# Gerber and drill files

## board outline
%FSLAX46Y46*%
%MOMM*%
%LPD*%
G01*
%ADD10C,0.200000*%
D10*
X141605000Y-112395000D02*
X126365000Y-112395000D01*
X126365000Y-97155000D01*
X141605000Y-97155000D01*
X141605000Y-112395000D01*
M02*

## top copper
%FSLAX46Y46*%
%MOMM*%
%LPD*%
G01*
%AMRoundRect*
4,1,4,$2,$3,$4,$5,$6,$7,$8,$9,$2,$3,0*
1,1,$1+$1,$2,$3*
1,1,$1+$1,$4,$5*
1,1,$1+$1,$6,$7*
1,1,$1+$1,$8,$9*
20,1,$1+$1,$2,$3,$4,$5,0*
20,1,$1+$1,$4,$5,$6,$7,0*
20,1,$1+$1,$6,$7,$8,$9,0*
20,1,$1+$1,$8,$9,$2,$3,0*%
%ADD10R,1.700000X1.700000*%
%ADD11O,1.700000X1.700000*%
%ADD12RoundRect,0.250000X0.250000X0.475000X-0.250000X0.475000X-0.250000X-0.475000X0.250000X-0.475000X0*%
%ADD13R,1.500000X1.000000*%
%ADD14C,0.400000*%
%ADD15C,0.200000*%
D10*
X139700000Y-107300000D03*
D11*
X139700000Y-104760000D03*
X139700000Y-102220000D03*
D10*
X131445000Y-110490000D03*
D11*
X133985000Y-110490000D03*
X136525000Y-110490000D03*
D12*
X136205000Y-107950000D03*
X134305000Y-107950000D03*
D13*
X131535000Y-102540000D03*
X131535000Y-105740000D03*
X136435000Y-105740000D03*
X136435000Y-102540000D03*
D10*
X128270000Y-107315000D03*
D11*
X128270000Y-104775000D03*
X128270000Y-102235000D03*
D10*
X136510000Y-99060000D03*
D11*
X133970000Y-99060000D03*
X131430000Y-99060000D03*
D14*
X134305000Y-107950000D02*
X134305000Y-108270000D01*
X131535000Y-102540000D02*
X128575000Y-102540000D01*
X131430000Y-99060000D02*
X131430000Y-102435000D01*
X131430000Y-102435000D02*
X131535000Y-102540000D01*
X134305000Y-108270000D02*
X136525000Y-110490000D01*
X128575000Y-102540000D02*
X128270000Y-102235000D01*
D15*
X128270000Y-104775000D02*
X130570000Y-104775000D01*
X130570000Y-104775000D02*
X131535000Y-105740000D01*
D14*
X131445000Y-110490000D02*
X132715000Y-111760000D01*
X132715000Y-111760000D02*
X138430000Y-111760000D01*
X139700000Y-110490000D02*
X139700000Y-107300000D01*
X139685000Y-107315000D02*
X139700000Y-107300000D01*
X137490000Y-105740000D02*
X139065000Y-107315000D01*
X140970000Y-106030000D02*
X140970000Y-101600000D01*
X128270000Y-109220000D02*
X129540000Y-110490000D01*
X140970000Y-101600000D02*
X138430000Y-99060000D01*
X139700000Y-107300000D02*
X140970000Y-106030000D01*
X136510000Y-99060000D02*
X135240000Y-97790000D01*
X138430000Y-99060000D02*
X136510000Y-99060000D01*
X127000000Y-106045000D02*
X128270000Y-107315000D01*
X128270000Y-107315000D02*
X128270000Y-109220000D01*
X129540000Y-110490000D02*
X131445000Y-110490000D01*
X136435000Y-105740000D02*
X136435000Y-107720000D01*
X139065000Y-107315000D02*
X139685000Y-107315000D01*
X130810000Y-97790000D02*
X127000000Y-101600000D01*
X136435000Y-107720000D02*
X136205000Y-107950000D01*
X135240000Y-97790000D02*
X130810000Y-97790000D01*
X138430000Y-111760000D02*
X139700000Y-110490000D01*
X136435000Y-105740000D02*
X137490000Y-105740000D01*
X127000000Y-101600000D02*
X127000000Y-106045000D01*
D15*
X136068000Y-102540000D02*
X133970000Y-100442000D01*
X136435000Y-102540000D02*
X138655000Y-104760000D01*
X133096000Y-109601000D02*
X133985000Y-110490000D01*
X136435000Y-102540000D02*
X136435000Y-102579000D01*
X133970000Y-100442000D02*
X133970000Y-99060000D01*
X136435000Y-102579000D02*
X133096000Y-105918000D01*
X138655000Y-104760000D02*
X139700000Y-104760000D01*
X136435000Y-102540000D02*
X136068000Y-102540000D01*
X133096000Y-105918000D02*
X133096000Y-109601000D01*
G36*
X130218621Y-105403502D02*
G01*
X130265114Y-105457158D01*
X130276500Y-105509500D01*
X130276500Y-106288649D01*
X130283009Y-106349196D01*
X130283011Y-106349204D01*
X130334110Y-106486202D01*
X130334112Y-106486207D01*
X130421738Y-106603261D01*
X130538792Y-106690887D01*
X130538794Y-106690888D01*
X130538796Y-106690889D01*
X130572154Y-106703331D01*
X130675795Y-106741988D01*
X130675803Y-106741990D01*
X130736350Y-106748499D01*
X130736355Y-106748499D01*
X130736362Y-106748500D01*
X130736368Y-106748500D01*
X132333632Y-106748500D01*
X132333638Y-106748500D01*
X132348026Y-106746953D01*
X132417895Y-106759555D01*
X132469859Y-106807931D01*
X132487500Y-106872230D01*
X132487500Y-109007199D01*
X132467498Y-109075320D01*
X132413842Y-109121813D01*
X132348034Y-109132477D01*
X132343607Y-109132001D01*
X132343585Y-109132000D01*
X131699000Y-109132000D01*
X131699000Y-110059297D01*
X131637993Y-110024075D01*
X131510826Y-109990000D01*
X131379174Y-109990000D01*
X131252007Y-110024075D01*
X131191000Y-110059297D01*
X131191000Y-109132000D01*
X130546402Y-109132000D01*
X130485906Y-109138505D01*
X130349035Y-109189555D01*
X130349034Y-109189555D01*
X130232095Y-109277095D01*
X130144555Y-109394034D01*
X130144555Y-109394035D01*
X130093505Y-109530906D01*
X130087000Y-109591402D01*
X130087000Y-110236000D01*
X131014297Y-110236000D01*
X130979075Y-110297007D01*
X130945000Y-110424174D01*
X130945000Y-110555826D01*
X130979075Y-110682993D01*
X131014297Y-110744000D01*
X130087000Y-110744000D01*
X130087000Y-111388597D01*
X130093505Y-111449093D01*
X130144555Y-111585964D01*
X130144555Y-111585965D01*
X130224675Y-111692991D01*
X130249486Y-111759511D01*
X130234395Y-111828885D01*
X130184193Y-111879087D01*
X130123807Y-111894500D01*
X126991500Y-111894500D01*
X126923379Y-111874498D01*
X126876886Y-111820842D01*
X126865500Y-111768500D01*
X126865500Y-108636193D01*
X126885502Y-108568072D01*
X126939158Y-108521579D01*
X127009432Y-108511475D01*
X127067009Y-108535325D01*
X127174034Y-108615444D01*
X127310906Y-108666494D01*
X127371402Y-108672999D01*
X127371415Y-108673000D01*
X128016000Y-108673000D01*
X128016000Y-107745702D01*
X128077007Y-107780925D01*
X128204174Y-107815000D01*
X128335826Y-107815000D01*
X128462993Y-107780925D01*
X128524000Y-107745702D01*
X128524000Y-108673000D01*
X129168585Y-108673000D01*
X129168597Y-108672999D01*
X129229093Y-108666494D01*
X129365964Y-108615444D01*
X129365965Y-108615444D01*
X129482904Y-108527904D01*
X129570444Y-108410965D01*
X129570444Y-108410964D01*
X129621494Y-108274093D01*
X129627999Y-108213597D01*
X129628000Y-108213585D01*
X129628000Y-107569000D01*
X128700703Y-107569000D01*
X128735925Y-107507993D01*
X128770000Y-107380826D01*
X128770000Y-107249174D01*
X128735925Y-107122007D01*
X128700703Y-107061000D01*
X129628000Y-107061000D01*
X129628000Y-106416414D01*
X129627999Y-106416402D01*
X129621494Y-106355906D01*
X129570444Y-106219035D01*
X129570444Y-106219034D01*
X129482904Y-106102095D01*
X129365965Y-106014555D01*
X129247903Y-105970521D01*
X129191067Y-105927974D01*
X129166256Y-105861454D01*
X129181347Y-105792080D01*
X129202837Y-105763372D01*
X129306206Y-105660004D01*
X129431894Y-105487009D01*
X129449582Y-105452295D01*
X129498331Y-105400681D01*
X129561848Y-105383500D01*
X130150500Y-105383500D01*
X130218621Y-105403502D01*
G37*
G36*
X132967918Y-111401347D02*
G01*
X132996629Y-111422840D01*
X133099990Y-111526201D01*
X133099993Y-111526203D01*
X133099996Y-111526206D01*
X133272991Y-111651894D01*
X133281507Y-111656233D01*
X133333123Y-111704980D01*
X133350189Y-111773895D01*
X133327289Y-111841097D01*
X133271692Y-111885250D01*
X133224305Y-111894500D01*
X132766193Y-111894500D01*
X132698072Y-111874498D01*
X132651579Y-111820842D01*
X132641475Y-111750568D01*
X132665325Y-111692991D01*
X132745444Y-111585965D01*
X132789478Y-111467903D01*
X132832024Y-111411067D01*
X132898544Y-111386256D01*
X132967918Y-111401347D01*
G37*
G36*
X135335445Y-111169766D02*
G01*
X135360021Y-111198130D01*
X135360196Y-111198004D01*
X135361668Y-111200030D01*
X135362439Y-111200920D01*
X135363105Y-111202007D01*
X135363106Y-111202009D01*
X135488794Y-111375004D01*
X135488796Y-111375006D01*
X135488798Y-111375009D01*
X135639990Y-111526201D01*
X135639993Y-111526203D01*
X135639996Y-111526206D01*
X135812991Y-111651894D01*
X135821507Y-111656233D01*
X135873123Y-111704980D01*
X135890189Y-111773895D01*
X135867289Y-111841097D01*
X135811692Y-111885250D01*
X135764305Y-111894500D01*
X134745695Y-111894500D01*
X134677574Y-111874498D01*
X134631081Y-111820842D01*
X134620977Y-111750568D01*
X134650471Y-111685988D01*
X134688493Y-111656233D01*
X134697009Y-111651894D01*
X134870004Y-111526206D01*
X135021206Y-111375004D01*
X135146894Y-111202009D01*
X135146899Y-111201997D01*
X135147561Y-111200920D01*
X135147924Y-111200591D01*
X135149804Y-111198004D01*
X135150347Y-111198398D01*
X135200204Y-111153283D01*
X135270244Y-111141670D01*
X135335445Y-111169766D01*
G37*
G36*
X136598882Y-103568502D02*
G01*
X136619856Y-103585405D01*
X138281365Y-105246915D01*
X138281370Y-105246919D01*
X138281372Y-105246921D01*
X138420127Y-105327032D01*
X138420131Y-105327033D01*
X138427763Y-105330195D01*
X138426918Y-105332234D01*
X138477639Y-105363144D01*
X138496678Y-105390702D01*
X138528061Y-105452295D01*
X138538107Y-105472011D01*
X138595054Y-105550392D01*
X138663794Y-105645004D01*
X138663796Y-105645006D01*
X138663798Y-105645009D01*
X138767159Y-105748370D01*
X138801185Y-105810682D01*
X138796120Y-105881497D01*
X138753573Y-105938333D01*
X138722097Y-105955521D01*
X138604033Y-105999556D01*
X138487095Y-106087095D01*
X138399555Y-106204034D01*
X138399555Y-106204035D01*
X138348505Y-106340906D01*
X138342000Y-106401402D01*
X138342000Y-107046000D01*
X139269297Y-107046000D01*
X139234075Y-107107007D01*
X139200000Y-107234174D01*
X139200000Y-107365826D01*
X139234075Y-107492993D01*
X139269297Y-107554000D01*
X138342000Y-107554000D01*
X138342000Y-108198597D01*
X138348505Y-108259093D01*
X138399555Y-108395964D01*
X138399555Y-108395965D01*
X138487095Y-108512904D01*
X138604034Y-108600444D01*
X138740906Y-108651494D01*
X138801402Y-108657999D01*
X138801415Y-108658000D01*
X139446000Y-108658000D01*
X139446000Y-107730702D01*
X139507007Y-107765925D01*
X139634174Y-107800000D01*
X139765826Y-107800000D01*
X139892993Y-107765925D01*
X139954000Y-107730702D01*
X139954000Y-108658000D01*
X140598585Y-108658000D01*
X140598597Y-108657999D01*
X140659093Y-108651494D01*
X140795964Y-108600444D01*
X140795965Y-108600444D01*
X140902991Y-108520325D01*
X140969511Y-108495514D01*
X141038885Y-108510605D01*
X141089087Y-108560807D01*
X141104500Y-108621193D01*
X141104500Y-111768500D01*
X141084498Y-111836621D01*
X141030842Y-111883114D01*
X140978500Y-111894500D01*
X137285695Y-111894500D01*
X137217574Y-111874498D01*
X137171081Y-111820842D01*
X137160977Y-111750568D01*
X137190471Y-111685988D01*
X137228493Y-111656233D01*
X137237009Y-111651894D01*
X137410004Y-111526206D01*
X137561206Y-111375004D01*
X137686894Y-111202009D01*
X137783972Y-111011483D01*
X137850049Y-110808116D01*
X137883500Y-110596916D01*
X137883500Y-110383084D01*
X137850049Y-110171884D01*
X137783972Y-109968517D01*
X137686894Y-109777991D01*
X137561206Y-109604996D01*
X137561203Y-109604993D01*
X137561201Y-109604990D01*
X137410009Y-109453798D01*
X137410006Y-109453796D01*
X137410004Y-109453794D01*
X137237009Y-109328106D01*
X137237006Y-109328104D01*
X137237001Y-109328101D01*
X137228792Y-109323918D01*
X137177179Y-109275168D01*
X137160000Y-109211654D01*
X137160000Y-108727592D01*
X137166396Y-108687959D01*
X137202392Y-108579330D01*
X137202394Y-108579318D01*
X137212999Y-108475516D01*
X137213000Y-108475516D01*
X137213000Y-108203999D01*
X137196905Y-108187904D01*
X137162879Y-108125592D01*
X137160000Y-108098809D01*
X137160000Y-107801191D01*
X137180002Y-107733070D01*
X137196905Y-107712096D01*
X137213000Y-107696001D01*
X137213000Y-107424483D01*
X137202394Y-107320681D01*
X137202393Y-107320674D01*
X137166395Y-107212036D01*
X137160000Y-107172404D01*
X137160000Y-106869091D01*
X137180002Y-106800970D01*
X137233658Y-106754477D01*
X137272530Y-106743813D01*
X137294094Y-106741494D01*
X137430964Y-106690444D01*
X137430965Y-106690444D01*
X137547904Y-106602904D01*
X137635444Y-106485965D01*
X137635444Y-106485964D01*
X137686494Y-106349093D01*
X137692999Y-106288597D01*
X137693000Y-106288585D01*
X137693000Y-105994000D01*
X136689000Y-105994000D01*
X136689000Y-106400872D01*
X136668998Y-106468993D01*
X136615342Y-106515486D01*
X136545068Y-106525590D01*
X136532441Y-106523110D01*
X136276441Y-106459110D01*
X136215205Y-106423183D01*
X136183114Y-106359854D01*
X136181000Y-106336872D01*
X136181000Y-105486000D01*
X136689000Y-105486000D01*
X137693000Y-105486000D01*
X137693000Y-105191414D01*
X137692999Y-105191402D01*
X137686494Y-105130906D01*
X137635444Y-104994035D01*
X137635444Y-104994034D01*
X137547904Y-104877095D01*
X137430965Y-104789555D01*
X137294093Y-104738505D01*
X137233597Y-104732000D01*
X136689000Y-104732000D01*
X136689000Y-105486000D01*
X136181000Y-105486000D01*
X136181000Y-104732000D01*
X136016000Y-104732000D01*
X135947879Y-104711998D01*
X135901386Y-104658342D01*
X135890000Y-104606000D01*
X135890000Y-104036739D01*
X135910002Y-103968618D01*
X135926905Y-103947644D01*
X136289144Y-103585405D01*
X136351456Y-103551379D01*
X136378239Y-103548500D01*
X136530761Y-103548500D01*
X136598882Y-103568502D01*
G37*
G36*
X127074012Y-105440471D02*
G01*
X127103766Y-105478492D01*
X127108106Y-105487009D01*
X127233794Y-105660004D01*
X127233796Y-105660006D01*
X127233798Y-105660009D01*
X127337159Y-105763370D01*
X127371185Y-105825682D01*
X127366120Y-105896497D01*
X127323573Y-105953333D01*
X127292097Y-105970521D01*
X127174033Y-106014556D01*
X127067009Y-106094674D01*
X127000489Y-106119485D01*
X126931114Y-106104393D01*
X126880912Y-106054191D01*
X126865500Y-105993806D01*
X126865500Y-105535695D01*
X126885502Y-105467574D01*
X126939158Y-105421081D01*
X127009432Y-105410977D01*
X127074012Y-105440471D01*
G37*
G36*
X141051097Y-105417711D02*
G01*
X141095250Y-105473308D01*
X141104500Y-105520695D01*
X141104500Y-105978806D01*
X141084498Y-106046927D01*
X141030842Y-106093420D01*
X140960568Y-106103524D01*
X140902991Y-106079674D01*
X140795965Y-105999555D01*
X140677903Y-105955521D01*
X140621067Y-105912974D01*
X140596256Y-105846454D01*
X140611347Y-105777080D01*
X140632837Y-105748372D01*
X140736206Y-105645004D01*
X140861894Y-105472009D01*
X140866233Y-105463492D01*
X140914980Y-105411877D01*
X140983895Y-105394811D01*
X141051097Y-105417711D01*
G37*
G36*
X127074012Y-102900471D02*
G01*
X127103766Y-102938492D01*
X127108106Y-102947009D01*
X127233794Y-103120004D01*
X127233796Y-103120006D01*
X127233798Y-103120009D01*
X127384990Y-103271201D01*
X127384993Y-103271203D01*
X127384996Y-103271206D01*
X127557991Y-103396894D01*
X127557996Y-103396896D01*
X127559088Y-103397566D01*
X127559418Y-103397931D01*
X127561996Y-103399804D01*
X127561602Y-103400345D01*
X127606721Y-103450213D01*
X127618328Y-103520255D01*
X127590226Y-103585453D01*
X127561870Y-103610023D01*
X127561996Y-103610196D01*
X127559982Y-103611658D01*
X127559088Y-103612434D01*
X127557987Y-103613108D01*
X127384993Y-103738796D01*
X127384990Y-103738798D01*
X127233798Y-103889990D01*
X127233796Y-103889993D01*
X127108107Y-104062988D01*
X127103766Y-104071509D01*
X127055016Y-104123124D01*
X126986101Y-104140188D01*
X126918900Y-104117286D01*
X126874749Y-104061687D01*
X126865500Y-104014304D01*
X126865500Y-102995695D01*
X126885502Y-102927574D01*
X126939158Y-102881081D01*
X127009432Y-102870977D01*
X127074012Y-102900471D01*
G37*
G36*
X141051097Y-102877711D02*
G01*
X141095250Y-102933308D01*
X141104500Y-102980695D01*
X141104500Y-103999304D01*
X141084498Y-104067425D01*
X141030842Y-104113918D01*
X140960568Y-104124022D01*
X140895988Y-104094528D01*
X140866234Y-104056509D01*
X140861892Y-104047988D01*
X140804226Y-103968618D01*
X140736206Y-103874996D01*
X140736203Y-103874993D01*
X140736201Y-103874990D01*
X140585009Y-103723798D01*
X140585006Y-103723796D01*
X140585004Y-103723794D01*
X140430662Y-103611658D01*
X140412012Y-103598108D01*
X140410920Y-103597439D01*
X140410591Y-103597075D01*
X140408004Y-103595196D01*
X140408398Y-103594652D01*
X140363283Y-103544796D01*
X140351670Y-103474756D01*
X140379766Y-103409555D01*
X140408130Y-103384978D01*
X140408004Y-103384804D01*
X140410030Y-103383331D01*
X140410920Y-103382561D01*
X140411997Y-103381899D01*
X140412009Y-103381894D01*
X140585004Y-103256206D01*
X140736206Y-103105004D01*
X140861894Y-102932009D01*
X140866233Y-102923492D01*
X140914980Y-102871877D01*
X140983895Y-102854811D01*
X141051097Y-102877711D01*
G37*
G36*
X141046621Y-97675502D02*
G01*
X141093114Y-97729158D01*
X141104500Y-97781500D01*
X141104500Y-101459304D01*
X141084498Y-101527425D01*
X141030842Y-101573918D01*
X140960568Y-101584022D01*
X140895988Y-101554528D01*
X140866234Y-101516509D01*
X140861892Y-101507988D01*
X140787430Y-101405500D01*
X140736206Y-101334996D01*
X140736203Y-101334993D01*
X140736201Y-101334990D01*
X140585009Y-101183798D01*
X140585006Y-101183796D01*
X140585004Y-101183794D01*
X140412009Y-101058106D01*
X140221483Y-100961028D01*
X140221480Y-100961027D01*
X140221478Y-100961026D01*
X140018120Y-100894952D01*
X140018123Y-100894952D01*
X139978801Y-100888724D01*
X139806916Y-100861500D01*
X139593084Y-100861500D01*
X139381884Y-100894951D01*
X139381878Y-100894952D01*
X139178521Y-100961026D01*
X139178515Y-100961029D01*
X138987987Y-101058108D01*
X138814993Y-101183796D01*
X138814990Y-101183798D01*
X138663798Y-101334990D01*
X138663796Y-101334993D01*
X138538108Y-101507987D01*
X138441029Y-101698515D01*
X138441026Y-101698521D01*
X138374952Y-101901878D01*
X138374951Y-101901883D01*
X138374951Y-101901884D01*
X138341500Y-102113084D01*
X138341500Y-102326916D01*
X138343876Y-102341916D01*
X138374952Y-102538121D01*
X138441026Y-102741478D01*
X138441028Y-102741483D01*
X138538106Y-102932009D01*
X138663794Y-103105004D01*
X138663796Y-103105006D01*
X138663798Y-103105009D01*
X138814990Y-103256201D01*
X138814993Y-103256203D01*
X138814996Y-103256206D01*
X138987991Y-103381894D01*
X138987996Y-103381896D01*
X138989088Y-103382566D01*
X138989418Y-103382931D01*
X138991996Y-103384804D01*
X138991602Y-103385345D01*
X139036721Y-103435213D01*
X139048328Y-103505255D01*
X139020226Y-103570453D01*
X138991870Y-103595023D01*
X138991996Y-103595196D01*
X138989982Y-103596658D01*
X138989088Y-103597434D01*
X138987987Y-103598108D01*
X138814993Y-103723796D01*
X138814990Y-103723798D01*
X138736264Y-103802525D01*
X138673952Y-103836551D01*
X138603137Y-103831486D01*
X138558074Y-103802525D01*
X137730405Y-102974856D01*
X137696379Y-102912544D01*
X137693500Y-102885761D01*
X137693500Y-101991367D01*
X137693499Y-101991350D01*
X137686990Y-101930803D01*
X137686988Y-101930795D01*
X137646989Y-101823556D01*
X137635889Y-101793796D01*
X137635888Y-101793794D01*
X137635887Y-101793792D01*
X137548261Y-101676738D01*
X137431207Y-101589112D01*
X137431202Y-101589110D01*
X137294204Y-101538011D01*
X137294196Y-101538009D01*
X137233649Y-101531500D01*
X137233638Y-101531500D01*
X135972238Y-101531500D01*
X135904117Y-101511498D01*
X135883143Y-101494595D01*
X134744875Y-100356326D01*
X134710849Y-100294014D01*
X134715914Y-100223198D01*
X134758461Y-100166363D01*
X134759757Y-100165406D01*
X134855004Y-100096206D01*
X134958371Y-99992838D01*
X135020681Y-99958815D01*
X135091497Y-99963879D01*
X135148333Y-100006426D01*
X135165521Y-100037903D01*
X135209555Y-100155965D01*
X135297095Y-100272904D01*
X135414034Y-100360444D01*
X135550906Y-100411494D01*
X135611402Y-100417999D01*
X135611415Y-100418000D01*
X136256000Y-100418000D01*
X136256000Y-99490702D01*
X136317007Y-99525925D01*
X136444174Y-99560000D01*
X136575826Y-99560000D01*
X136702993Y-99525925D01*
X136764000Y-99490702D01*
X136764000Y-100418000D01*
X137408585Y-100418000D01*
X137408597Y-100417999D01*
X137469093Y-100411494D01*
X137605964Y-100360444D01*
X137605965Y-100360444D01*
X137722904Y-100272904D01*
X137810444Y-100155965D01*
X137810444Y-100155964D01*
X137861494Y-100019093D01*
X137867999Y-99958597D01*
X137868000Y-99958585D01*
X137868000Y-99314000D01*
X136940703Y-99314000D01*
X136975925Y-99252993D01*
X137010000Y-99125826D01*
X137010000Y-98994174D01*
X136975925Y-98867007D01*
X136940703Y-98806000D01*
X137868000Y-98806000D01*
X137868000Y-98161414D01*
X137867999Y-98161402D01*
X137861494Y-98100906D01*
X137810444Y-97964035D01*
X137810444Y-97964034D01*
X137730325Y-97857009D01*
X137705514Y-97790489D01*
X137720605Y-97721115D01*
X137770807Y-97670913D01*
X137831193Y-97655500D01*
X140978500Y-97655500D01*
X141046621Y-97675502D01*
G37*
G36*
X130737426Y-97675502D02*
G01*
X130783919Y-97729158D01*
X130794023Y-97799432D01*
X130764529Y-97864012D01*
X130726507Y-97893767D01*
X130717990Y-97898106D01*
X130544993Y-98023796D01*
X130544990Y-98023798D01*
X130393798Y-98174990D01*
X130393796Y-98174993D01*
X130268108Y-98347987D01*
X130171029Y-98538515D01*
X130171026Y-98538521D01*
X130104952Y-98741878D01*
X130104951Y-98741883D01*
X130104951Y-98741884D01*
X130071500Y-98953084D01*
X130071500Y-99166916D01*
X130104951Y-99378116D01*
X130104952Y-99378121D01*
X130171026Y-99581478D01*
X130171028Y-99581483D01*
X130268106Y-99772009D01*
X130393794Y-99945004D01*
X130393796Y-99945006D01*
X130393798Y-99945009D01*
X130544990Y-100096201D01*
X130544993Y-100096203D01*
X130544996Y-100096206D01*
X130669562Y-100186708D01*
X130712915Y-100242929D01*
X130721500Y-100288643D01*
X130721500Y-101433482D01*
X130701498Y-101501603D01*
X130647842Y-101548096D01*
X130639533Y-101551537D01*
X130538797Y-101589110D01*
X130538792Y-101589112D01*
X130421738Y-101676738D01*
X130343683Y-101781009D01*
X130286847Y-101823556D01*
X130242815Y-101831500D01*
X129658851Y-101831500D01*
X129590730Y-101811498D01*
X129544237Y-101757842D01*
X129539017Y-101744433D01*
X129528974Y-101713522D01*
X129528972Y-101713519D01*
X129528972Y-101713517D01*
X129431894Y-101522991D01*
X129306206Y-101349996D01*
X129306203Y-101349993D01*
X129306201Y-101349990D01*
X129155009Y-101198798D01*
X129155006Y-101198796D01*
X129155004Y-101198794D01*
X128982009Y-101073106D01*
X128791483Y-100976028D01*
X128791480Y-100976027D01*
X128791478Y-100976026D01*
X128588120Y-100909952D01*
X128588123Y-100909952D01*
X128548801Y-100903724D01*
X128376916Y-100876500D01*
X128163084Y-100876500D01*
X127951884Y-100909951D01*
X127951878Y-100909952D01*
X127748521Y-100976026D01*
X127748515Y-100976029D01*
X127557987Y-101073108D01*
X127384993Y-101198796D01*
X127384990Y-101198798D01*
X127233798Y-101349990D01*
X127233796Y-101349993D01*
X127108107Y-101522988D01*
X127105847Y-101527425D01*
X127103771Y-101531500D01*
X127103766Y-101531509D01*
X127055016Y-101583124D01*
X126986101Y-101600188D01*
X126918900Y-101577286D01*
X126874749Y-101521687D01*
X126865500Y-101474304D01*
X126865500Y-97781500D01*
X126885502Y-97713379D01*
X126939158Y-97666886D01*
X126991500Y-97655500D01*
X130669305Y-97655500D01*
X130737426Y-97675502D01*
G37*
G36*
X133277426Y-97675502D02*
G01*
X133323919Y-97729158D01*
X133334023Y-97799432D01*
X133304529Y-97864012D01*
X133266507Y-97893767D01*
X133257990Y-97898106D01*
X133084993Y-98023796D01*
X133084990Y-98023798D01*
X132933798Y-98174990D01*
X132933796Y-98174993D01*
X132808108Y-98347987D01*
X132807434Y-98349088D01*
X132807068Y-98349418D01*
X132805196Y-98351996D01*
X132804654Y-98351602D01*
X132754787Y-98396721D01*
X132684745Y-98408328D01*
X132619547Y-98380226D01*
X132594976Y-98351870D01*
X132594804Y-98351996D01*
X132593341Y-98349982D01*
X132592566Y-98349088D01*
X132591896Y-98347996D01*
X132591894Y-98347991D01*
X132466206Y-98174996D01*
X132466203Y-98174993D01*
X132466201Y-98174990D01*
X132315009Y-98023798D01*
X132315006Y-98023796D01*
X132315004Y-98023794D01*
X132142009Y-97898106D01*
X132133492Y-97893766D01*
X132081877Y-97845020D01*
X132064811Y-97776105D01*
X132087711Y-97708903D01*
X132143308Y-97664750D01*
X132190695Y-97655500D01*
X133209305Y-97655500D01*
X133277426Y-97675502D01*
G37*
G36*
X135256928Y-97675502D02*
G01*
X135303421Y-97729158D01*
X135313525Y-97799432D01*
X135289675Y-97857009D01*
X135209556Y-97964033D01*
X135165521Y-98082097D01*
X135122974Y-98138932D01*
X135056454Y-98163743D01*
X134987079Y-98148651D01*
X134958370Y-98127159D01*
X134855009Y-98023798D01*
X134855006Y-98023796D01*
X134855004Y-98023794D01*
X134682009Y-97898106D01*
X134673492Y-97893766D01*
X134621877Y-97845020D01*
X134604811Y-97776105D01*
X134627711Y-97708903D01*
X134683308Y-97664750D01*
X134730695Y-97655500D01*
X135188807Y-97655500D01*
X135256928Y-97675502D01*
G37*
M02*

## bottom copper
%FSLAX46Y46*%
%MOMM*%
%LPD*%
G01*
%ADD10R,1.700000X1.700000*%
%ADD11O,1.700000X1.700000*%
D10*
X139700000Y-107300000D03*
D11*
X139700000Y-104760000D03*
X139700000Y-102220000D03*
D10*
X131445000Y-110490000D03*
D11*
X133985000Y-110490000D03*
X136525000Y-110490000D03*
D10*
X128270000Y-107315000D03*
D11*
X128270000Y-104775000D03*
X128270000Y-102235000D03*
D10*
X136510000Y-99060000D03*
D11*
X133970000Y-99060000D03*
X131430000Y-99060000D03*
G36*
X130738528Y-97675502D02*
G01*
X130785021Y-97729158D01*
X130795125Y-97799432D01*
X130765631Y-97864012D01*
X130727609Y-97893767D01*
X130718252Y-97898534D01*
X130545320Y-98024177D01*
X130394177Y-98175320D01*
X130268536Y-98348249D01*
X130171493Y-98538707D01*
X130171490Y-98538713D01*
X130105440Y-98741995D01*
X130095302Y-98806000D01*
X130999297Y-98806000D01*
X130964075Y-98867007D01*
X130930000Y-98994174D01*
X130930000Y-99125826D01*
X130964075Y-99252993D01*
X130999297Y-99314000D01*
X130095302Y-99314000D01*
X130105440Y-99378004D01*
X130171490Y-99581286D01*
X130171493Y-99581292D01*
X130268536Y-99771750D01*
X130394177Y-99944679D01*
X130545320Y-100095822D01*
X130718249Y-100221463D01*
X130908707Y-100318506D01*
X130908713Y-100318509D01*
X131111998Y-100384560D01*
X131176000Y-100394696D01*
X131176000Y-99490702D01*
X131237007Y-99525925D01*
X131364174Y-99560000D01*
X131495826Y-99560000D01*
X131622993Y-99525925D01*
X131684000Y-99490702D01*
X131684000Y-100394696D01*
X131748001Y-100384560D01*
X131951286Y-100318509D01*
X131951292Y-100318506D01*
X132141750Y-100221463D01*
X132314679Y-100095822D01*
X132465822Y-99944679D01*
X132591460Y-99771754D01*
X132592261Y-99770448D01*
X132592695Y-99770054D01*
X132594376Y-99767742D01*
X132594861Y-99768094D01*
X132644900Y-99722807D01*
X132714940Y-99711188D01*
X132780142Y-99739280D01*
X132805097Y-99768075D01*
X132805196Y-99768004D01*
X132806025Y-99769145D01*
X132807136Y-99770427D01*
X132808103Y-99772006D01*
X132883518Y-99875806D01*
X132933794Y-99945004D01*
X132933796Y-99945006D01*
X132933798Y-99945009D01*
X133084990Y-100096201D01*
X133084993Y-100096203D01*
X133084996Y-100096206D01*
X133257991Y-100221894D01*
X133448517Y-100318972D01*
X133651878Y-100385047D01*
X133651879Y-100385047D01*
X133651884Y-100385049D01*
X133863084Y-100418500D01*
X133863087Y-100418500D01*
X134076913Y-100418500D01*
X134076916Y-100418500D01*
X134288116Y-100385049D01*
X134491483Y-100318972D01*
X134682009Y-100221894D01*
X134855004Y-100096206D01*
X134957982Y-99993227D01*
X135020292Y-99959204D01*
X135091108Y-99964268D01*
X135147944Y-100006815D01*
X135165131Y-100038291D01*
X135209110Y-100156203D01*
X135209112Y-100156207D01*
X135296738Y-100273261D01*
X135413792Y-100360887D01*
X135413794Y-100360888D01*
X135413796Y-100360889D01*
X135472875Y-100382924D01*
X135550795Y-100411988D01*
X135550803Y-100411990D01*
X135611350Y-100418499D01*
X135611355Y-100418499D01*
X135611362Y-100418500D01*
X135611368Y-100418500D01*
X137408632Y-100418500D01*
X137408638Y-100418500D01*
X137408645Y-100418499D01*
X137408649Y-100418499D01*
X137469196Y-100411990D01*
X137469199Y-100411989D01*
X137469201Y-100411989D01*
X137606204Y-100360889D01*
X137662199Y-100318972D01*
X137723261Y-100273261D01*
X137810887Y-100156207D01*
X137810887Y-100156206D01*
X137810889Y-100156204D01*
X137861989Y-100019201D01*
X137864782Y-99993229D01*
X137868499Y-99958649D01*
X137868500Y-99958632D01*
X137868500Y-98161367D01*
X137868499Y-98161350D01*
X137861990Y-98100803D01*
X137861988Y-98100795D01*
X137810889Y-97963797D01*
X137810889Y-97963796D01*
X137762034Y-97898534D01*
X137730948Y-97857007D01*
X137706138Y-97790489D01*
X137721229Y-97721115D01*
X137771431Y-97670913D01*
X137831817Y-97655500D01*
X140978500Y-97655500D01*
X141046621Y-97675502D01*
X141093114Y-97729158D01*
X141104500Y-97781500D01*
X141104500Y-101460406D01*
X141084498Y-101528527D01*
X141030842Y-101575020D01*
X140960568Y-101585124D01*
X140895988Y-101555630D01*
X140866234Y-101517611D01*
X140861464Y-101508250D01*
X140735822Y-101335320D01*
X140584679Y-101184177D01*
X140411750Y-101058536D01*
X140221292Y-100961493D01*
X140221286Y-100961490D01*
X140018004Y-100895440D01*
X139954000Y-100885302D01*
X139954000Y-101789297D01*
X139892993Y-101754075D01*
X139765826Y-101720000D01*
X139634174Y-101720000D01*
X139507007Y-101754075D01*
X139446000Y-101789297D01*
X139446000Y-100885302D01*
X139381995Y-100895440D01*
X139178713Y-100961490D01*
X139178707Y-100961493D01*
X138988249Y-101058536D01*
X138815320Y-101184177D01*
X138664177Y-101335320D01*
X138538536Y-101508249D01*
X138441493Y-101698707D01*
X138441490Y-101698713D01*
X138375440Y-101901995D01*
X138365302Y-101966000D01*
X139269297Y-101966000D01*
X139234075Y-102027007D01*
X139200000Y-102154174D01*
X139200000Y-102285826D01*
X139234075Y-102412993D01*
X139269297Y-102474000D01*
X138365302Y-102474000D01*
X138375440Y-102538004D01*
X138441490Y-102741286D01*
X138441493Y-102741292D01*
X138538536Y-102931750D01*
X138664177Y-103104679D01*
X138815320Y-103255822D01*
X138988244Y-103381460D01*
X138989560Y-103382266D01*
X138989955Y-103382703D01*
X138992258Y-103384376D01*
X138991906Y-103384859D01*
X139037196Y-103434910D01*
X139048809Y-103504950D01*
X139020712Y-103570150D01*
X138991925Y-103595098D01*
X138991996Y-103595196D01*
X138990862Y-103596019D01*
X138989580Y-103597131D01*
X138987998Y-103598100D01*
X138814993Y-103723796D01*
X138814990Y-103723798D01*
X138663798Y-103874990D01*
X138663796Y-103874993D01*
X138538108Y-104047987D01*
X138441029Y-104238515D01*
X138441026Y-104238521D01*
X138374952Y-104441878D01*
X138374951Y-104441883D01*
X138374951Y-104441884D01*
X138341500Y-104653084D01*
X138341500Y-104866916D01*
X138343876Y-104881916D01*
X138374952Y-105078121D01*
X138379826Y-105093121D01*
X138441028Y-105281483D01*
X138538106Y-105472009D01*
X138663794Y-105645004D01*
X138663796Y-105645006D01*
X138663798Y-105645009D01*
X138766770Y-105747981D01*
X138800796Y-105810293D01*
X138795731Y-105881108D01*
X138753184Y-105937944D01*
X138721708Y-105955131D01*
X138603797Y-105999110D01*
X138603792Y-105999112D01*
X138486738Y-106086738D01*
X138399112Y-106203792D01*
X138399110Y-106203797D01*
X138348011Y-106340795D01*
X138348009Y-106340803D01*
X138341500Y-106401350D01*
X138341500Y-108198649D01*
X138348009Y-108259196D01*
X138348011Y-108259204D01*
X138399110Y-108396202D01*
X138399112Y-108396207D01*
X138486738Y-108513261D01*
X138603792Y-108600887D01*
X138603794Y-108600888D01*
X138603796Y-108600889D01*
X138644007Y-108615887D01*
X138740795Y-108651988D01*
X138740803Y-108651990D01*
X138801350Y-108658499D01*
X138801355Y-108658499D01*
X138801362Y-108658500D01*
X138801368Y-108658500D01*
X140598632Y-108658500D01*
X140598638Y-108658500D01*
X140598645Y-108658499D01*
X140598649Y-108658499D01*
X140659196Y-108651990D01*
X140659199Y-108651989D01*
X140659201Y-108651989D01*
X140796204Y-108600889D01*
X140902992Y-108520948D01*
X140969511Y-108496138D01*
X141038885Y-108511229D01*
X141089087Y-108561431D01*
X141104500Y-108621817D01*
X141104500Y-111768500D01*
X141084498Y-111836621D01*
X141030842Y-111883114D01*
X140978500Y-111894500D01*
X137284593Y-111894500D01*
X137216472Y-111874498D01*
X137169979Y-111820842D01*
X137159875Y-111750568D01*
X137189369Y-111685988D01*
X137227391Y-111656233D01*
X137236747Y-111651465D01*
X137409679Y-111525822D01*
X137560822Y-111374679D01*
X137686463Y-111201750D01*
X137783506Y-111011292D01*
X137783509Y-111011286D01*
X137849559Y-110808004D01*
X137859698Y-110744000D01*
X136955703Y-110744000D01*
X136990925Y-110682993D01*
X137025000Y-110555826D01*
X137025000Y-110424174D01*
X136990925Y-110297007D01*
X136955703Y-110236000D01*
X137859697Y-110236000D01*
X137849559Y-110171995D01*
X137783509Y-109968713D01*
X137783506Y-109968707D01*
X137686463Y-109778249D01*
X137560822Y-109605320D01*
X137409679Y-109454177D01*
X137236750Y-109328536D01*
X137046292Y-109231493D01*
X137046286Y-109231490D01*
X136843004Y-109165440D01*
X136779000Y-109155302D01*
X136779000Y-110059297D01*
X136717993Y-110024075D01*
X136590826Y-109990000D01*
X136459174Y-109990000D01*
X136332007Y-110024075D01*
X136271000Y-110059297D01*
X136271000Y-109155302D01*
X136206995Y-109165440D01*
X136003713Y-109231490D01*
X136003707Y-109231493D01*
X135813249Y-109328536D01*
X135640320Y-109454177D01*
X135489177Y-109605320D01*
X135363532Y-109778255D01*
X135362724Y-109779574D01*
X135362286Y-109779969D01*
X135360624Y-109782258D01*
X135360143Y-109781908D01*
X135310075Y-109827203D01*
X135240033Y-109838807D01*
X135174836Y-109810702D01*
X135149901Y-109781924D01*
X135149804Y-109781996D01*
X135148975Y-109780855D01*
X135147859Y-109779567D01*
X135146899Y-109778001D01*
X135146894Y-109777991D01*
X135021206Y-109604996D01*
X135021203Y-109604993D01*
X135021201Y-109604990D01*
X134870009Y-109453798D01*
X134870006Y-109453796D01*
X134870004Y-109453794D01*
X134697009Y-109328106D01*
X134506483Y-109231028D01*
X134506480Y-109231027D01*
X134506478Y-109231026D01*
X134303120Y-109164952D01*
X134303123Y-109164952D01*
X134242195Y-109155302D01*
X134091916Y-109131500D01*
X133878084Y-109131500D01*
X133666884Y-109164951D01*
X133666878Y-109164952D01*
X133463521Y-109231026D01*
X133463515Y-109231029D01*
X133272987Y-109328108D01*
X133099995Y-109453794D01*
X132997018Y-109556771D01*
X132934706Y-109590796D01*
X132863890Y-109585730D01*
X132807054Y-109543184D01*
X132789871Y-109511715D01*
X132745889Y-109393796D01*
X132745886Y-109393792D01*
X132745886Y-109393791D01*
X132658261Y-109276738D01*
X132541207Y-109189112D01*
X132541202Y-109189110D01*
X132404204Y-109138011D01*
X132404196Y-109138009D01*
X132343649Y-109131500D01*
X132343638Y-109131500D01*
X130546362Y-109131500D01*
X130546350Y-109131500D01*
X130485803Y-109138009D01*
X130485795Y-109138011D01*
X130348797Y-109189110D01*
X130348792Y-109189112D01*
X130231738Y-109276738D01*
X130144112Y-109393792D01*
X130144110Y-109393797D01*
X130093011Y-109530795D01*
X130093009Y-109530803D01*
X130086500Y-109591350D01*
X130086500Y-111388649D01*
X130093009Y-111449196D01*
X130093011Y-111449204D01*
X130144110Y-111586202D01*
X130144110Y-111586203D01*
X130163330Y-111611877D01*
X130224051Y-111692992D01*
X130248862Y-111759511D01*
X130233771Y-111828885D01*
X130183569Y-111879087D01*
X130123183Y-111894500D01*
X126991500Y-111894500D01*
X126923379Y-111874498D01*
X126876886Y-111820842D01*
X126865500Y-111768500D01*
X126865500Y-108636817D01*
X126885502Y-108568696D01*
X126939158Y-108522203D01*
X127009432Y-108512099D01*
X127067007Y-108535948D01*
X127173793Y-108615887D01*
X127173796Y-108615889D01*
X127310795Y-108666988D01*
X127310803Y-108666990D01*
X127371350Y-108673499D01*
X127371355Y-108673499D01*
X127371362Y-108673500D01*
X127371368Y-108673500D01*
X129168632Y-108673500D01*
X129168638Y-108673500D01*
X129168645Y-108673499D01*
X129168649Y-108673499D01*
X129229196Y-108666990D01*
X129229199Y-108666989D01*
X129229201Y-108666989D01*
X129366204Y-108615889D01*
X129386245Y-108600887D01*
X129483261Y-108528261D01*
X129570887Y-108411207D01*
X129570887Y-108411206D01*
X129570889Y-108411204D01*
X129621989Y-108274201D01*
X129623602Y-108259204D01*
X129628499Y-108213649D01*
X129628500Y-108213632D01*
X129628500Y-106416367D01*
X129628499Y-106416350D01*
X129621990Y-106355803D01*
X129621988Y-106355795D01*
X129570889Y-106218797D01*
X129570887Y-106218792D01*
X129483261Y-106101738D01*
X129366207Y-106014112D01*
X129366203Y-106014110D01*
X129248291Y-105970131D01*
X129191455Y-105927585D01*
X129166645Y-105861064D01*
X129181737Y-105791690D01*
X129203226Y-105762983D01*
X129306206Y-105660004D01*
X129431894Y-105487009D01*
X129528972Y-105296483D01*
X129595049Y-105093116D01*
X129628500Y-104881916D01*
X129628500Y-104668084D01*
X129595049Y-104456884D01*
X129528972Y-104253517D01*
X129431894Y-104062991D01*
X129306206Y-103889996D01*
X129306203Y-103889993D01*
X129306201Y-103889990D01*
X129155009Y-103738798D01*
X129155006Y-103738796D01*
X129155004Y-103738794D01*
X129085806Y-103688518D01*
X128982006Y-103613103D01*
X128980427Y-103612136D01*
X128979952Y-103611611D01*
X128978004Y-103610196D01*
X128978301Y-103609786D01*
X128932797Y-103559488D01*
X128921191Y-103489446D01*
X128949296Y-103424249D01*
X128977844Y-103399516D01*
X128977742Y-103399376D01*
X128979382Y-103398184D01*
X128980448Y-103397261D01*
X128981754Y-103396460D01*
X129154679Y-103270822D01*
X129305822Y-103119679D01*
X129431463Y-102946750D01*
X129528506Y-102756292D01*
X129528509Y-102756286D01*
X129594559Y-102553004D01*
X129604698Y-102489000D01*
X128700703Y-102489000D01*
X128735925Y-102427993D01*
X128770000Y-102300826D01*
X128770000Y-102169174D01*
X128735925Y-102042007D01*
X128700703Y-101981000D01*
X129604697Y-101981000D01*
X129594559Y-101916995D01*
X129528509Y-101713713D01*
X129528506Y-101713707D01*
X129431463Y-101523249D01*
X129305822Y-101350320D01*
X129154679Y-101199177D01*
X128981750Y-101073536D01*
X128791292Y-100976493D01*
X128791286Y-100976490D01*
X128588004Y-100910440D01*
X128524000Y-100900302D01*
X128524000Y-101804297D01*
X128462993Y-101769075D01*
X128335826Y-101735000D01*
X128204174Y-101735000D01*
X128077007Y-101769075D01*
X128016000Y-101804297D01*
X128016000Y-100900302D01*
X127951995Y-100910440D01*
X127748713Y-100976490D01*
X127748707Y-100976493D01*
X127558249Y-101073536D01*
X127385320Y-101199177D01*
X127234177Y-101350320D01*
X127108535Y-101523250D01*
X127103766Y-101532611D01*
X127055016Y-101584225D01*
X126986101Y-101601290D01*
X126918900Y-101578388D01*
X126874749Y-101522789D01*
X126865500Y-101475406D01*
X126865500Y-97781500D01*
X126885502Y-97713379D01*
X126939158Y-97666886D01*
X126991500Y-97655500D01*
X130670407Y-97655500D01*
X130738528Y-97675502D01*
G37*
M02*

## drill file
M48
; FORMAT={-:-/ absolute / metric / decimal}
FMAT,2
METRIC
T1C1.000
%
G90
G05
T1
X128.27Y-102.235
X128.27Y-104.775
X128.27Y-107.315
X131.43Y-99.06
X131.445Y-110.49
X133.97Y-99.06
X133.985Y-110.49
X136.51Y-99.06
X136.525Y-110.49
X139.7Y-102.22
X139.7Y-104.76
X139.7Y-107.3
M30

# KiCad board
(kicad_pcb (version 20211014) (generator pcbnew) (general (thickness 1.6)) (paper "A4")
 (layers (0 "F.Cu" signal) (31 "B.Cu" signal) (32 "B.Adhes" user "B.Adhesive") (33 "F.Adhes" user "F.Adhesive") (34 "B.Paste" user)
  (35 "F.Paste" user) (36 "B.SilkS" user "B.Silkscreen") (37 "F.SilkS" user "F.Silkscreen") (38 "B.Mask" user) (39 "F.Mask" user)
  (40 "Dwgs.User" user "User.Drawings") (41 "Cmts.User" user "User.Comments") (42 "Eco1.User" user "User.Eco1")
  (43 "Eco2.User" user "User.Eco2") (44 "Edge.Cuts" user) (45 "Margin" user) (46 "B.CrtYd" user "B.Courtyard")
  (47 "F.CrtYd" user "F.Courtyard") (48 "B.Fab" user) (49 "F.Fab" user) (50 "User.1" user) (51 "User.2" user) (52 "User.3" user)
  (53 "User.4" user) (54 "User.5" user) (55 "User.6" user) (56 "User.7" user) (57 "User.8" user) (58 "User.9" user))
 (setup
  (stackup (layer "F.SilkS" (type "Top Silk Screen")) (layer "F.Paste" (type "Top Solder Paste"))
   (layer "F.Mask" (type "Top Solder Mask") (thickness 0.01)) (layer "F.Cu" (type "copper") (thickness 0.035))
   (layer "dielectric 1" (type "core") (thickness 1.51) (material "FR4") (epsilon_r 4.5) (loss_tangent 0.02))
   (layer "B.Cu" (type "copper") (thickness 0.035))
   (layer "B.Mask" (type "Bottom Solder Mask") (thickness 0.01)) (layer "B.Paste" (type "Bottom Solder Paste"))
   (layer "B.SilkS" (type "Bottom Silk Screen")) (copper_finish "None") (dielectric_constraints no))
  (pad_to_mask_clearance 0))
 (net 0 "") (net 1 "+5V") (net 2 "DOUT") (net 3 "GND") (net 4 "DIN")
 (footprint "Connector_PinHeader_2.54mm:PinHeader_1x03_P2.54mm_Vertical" (layer "F.Cu") (at 139.7 107.3 180)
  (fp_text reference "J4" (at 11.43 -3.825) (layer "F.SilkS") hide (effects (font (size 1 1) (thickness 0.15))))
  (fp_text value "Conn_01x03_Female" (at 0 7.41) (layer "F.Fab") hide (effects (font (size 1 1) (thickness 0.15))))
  (pad "1" thru_hole rect (at 0 0 180) (size 1.7 1.7) (drill 1) (layers *.Cu *.Mask) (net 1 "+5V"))
  (pad "2" thru_hole oval (at 0 2.54 180) (size 1.7 1.7) (drill 1) (layers *.Cu *.Mask) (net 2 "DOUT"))
  (pad "3" thru_hole oval (at 0 5.08 180) (size 1.7 1.7) (drill 1) (layers *.Cu *.Mask) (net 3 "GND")))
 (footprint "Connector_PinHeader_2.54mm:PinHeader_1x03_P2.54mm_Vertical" (layer "F.Cu") (at 131.445 110.49 90)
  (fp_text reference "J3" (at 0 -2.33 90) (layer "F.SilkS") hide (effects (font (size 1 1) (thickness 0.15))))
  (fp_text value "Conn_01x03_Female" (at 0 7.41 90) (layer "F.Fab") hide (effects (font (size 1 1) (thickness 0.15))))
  (pad "1" thru_hole rect (at 0 0 90) (size 1.7 1.7) (drill 1) (layers *.Cu *.Mask) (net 1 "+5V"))
  (pad "2" thru_hole oval (at 0 2.54 90) (size 1.7 1.7) (drill 1) (layers *.Cu *.Mask) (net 2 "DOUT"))
  (pad "3" thru_hole oval (at 0 5.08 90) (size 1.7 1.7) (drill 1) (layers *.Cu *.Mask) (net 3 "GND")))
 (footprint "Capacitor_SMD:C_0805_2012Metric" (layer "F.Cu") (at 135.255 107.95 180)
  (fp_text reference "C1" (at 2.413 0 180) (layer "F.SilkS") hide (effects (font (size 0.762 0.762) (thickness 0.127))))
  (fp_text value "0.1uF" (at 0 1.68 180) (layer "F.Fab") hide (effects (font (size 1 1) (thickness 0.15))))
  (pad "1" smd roundrect (at -0.95 0 180) (size 1 1.45) (layers "F.Cu" "F.Paste" "F.Mask") (roundrect_rratio 0.25) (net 1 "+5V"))
  (pad "2" smd roundrect (at 0.95 0 180) (size 1 1.45) (layers "F.Cu" "F.Paste" "F.Mask") (roundrect_rratio 0.25) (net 3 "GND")))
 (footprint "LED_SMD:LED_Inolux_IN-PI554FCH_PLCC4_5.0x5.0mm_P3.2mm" (layer "F.Cu") (at 133.985 104.14)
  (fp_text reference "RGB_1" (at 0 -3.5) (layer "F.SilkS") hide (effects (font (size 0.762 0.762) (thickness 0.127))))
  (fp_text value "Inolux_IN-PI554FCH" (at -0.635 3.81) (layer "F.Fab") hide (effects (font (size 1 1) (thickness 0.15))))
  (pad "1" smd rect (at -2.45 -1.6) (size 1.5 1) (layers "F.Cu" "F.Paste" "F.Mask") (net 3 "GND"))
  (pad "2" smd rect (at -2.45 1.6) (size 1.5 1) (layers "F.Cu" "F.Paste" "F.Mask") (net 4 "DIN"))
  (pad "3" smd rect (at 2.45 1.6) (size 1.5 1) (layers "F.Cu" "F.Paste" "F.Mask") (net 1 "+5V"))
  (pad "4" smd rect (at 2.45 -1.6) (size 1.5 1) (layers "F.Cu" "F.Paste" "F.Mask") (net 2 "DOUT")))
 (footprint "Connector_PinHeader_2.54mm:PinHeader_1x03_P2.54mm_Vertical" (layer "F.Cu") (at 128.27 107.315 180)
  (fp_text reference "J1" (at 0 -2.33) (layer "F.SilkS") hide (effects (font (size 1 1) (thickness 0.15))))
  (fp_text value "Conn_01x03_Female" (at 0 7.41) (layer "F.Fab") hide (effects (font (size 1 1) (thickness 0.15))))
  (pad "1" thru_hole rect (at 0 0 180) (size 1.7 1.7) (drill 1) (layers *.Cu *.Mask) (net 1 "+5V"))
  (pad "2" thru_hole oval (at 0 2.54 180) (size 1.7 1.7) (drill 1) (layers *.Cu *.Mask) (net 4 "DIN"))
  (pad "3" thru_hole oval (at 0 5.08 180) (size 1.7 1.7) (drill 1) (layers *.Cu *.Mask) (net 3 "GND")))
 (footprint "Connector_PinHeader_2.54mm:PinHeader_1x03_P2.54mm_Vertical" (layer "F.Cu") (at 136.51 99.06 -90)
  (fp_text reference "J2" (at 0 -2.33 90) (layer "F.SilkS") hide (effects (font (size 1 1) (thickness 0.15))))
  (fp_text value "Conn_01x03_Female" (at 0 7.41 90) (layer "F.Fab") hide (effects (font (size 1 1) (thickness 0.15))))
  (pad "1" thru_hole rect (at 0 0 270) (size 1.7 1.7) (drill 1) (layers *.Cu *.Mask) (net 1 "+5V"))
  (pad "2" thru_hole oval (at 0 2.54 270) (size 1.7 1.7) (drill 1) (layers *.Cu *.Mask) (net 2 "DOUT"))
  (pad "3" thru_hole oval (at 0 5.08 270) (size 1.7 1.7) (drill 1) (layers *.Cu *.Mask) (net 3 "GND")))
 (gr_poly
  (pts (xy 141.605 112.395) (xy 126.365 112.395) (xy 126.365 97.155) (xy 141.605 97.155)) (layer "Edge.Cuts") (width 0.2) (fill none))
 (segment (start 134.305 107.95) (end 134.305 108.27) (width 0.4) (layer "F.Cu") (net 3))
 (segment (start 131.535 102.54) (end 128.575 102.54) (width 0.4) (layer "F.Cu") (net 3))
 (segment (start 131.43 99.06) (end 131.43 102.435) (width 0.4) (layer "F.Cu") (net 3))
 (segment (start 131.43 102.435) (end 131.535 102.54) (width 0.4) (layer "F.Cu") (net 3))
 (segment (start 134.305 108.27) (end 136.525 110.49) (width 0.4) (layer "F.Cu") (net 3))
 (segment (start 128.575 102.54) (end 128.27 102.235) (width 0.4) (layer "F.Cu") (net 3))
 (segment (start 128.27 104.775) (end 130.57 104.775) (width 0.2) (layer "F.Cu") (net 4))
 (segment (start 130.57 104.775) (end 131.535 105.74) (width 0.2) (layer "F.Cu") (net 4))
 (segment (start 131.445 110.49) (end 132.715 111.76) (width 0.4) (layer "F.Cu") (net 1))
 (segment (start 132.715 111.76) (end 138.43 111.76) (width 0.4) (layer "F.Cu") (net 1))
 (segment (start 139.7 110.49) (end 139.7 107.3) (width 0.4) (layer "F.Cu") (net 1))
 (segment (start 139.685 107.315) (end 139.7 107.3) (width 0.4) (layer "F.Cu") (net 1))
 (segment (start 137.49 105.74) (end 139.065 107.315) (width 0.4) (layer "F.Cu") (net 1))
 (segment (start 140.97 106.03) (end 140.97 101.6) (width 0.4) (layer "F.Cu") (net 1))
 (segment (start 128.27 109.22) (end 129.54 110.49) (width 0.4) (layer "F.Cu") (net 1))
 (segment (start 140.97 101.6) (end 138.43 99.06) (width 0.4) (layer "F.Cu") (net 1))
 (segment (start 139.7 107.3) (end 140.97 106.03) (width 0.4) (layer "F.Cu") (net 1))
 (segment (start 136.51 99.06) (end 135.24 97.79) (width 0.4) (layer "F.Cu") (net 1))
 (segment (start 138.43 99.06) (end 136.51 99.06) (width 0.4) (layer "F.Cu") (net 1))
 (segment (start 127 106.045) (end 128.27 107.315) (width 0.4) (layer "F.Cu") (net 1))
 (segment (start 128.27 107.315) (end 128.27 109.22) (width 0.4) (layer "F.Cu") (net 1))
 (segment (start 129.54 110.49) (end 131.445 110.49) (width 0.4) (layer "F.Cu") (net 1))
 (segment (start 136.435 105.74) (end 136.435 107.72) (width 0.4) (layer "F.Cu") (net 1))
 (segment (start 139.065 107.315) (end 139.685 107.315) (width 0.4) (layer "F.Cu") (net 1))
 (segment (start 130.81 97.79) (end 127 101.6) (width 0.4) (layer "F.Cu") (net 1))
 (segment (start 136.435 107.72) (end 136.205 107.95) (width 0.4) (layer "F.Cu") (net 1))
 (segment (start 135.24 97.79) (end 130.81 97.79) (width 0.4) (layer "F.Cu") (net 1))
 (segment (start 138.43 111.76) (end 139.7 110.49) (width 0.4) (layer "F.Cu") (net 1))
 (segment (start 136.435 105.74) (end 137.49 105.74) (width 0.4) (layer "F.Cu") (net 1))
 (segment (start 127 101.6) (end 127 106.045) (width 0.4) (layer "F.Cu") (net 1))
 (segment (start 136.068 102.54) (end 133.97 100.442) (width 0.2) (layer "F.Cu") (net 2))
 (segment (start 136.435 102.54) (end 138.655 104.76) (width 0.2) (layer "F.Cu") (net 2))
 (segment (start 133.096 109.601) (end 133.985 110.49) (width 0.2) (layer "F.Cu") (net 2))
 (segment (start 136.435 102.54) (end 136.435 102.579) (width 0.2) (layer "F.Cu") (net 2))
 (segment (start 133.97 100.442) (end 133.97 99.06) (width 0.2) (layer "F.Cu") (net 2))
 (segment (start 136.435 102.579) (end 133.096 105.918) (width 0.2) (layer "F.Cu") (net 2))
 (segment (start 138.655 104.76) (end 139.7 104.76) (width 0.2) (layer "F.Cu") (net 2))
 (segment (start 136.435 102.54) (end 136.068 102.54) (width 0.2) (layer "F.Cu") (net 2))
 (segment (start 133.096 105.918) (end 133.096 109.601) (width 0.2) (layer "F.Cu") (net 2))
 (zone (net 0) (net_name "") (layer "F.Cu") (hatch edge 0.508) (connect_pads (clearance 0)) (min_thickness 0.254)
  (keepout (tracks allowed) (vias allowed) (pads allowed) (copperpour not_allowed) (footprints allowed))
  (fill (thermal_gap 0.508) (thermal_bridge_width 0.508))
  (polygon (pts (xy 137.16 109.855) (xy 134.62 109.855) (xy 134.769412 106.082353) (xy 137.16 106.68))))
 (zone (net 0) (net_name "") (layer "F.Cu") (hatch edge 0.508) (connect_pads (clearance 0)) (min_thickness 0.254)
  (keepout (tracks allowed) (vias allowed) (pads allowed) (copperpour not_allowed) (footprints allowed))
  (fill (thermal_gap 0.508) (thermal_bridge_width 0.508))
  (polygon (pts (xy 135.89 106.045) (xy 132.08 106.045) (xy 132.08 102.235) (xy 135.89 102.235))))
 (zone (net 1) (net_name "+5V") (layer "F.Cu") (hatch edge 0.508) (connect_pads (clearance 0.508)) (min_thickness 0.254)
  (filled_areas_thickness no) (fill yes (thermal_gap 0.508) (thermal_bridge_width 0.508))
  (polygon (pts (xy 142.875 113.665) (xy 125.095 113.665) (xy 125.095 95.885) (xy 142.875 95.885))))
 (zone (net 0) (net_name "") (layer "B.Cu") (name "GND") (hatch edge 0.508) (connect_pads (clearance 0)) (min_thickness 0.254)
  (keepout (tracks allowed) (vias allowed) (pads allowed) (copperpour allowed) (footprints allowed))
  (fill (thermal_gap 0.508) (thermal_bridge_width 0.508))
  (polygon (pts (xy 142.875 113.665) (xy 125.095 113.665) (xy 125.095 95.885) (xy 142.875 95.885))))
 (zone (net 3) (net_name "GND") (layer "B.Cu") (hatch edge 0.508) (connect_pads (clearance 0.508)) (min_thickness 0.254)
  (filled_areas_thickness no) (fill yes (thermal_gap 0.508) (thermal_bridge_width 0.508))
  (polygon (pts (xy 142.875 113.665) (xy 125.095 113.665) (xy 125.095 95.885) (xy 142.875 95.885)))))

